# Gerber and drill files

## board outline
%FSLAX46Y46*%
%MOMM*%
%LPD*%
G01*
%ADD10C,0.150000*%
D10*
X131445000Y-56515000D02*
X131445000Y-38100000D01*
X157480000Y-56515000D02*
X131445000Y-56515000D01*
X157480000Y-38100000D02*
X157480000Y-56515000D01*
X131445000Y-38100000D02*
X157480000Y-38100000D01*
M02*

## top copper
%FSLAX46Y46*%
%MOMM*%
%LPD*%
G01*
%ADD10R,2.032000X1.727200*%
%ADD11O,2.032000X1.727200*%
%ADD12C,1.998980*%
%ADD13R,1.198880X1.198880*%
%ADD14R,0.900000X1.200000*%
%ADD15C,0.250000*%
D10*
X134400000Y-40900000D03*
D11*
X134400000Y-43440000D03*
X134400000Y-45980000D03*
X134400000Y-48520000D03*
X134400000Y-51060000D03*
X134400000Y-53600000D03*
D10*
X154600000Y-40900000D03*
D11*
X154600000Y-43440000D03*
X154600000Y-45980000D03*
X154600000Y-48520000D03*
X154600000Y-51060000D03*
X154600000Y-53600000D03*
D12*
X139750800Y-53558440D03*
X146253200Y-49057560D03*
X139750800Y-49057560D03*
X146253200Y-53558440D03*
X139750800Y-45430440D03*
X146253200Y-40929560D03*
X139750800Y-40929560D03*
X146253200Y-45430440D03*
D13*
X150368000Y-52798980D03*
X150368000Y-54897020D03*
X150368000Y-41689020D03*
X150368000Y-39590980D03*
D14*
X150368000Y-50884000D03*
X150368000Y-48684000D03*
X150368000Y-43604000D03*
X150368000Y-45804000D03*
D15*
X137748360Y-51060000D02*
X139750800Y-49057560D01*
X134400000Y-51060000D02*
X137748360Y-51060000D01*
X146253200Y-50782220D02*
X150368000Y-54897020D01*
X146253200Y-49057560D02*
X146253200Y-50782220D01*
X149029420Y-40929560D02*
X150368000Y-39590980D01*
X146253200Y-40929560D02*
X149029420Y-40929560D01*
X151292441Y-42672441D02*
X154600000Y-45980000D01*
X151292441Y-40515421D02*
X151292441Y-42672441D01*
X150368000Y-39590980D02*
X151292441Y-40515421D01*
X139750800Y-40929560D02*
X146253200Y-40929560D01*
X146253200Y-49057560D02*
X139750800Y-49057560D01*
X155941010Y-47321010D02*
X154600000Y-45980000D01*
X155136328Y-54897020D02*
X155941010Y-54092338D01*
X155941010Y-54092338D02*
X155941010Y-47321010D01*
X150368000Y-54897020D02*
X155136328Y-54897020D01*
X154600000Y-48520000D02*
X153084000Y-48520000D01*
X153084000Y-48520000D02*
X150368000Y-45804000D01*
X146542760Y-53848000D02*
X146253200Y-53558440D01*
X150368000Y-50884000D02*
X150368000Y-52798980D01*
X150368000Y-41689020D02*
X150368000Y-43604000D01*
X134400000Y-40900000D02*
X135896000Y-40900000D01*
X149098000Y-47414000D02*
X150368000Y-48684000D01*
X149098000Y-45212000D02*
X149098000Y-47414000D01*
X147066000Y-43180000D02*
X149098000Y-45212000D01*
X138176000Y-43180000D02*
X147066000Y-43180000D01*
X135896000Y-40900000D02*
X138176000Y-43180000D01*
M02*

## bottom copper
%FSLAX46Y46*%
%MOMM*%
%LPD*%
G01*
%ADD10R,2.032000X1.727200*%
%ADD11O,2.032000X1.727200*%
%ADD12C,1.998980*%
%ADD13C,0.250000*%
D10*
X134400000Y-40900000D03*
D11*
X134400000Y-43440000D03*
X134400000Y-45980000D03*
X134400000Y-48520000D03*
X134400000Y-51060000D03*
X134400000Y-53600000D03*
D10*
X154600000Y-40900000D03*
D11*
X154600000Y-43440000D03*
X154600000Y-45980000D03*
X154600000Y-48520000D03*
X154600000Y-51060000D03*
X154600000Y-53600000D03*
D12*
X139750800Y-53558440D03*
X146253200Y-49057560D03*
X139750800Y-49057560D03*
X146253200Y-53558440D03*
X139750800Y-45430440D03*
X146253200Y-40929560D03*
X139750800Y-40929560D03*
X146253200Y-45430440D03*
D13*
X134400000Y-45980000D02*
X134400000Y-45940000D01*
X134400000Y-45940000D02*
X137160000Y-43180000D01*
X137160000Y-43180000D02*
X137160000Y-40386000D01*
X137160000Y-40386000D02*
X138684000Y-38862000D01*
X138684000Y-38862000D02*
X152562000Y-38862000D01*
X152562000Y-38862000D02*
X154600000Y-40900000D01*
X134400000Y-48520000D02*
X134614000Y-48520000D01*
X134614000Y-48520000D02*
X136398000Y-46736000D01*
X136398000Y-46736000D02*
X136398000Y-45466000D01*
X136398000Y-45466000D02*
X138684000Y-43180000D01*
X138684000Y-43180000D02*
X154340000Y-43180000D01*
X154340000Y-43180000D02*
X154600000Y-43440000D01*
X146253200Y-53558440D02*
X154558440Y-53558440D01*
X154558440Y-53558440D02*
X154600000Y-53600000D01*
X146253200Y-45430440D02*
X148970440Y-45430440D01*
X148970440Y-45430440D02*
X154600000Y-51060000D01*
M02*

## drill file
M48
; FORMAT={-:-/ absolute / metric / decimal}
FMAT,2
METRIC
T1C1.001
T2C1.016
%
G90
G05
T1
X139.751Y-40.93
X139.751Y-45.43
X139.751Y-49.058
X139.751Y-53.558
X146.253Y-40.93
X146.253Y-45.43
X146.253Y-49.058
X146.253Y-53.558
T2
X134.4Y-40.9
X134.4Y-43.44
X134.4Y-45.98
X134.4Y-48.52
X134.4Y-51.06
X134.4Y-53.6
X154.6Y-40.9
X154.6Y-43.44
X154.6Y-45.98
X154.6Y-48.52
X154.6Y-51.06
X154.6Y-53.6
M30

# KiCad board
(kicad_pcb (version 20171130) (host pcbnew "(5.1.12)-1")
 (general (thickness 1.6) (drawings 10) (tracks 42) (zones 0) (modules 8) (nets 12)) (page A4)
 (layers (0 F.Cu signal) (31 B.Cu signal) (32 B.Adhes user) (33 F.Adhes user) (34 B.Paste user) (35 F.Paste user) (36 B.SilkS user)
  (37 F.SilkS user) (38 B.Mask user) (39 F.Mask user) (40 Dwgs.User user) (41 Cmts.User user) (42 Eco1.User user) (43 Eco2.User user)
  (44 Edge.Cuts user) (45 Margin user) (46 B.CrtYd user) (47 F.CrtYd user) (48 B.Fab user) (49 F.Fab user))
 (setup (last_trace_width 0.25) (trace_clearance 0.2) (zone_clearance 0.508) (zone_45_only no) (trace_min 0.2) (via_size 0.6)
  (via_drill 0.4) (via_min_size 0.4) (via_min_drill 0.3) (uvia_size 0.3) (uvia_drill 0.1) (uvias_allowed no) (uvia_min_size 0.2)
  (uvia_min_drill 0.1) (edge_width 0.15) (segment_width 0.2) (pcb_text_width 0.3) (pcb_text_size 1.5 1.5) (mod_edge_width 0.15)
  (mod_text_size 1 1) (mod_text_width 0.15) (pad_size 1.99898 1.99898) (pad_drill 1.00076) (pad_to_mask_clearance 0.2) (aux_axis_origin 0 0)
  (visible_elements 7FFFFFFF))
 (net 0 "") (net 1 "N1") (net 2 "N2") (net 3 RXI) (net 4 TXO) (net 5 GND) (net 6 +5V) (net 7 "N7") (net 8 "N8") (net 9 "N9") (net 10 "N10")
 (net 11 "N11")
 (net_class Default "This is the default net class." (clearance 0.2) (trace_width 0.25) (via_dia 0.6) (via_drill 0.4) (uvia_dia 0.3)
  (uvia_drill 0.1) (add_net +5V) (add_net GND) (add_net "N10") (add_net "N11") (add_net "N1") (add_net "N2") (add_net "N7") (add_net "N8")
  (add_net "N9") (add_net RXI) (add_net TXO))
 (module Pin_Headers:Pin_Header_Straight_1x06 (layer F.Cu) (at 134.4 40.9)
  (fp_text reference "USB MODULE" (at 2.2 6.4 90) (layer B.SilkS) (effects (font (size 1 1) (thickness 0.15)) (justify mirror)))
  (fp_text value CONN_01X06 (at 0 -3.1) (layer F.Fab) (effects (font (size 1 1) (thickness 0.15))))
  (pad 1 thru_hole rect (at 0 0) (size 2.032 1.7272) (drill 1.016) (layers *.Cu *.Mask F.SilkS) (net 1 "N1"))
  (pad 2 thru_hole oval (at 0 2.54) (size 2.032 1.7272) (drill 1.016) (layers *.Cu *.Mask F.SilkS) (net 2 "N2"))
  (pad 3 thru_hole oval (at 0 5.08) (size 2.032 1.7272) (drill 1.016) (layers *.Cu *.Mask F.SilkS) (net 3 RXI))
  (pad 4 thru_hole oval (at 0 7.62) (size 2.032 1.7272) (drill 1.016) (layers *.Cu *.Mask F.SilkS) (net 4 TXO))
  (pad 5 thru_hole oval (at 0 10.16) (size 2.032 1.7272) (drill 1.016) (layers *.Cu *.Mask F.SilkS) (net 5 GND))
  (pad 6 thru_hole oval (at 0 12.7) (size 2.032 1.7272) (drill 1.016) (layers *.Cu *.Mask F.SilkS) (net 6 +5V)))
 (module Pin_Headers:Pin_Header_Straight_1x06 (layer F.Cu) (at 154.6 40.9)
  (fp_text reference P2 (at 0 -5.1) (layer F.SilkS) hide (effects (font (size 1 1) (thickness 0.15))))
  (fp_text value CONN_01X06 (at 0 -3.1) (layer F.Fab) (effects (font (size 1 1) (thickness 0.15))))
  (pad 1 thru_hole rect (at 0 0) (size 2.032 1.7272) (drill 1.016) (layers *.Cu *.Mask F.SilkS) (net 3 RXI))
  (pad 2 thru_hole oval (at 0 2.54) (size 2.032 1.7272) (drill 1.016) (layers *.Cu *.Mask F.SilkS) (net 4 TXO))
  (pad 3 thru_hole oval (at 0 5.08) (size 2.032 1.7272) (drill 1.016) (layers *.Cu *.Mask F.SilkS) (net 5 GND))
  (pad 4 thru_hole oval (at 0 7.62) (size 2.032 1.7272) (drill 1.016) (layers *.Cu *.Mask F.SilkS) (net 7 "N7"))
  (pad 5 thru_hole oval (at 0 10.16) (size 2.032 1.7272) (drill 1.016) (layers *.Cu *.Mask F.SilkS) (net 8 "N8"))
  (pad 6 thru_hole oval (at 0 12.7) (size 2.032 1.7272) (drill 1.016) (layers *.Cu *.Mask F.SilkS) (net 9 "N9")))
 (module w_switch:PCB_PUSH (layer F.Cu) (at 143.002 51.308 90)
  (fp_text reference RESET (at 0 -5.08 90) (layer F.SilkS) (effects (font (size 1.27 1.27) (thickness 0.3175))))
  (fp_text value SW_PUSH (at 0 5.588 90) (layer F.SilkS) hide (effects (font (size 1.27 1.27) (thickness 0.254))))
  (pad 1 thru_hole circle (at -2.25044 -3.2512 90) (size 1.99898 1.99898) (drill 1.00076) (layers *.Cu *.Mask F.SilkS))
  (pad 2 thru_hole circle (at 2.25044 3.2512 90) (size 1.99898 1.99898) (drill 1.00076) (layers *.Cu *.Mask F.SilkS) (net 5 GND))
  (pad 4 thru_hole circle (at 2.25044 -3.2512 90) (size 1.99898 1.99898) (drill 1.00076) (layers *.Cu *.Mask F.SilkS) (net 5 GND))
  (pad 3 thru_hole circle (at -2.25044 3.2512 90) (size 1.99898 1.99898) (drill 1.00076) (layers *.Cu *.Mask F.SilkS) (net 9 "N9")))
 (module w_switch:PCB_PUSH (layer F.Cu) (at 143.002 43.18 90)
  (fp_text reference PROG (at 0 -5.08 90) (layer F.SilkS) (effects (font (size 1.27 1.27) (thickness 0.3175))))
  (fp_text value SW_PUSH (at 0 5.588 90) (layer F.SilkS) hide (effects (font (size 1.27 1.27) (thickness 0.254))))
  (pad 1 thru_hole circle (at -2.25044 -3.2512 90) (size 1.99898 1.99898) (drill 1.00076) (layers *.Cu *.Mask F.SilkS))
  (pad 2 thru_hole circle (at 2.25044 3.2512 90) (size 1.99898 1.99898) (drill 1.00076) (layers *.Cu *.Mask F.SilkS) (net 5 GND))
  (pad 4 thru_hole circle (at 2.25044 -3.2512 90) (size 1.99898 1.99898) (drill 1.00076) (layers *.Cu *.Mask F.SilkS) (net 5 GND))
  (pad 3 thru_hole circle (at -2.25044 3.2512 90) (size 1.99898 1.99898) (drill 1.00076) (layers *.Cu *.Mask F.SilkS) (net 8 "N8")))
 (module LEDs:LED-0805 (layer F.Cu) (at 150.368 53.848 90)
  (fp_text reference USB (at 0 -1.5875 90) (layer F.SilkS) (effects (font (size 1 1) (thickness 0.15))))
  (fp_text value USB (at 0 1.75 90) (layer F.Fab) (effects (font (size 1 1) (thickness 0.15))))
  (pad 2 smd rect (at 1.04902 0 270) (size 1.19888 1.19888) (layers F.Cu F.Paste F.Mask) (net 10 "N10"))
  (pad 1 smd rect (at -1.04902 0 270) (size 1.19888 1.19888) (layers F.Cu F.Paste F.Mask) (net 5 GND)))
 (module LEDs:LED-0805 (layer F.Cu) (at 150.368 40.64 270)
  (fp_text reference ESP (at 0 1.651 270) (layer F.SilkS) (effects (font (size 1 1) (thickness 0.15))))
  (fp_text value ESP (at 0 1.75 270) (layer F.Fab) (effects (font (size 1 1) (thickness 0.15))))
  (pad 2 smd rect (at 1.04902 0 90) (size 1.19888 1.19888) (layers F.Cu F.Paste F.Mask) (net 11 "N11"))
  (pad 1 smd rect (at -1.04902 0 90) (size 1.19888 1.19888) (layers F.Cu F.Paste F.Mask) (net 5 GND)))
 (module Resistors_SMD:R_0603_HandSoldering (layer F.Cu) (at 150.368 49.784 90)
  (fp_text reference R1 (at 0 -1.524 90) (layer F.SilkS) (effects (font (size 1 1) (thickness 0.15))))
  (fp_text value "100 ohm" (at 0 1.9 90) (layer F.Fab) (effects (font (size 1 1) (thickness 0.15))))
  (pad 1 smd rect (at -1.1 0 90) (size 1.2 0.9) (layers F.Cu F.Paste F.Mask) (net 10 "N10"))
  (pad 2 smd rect (at 1.1 0 90) (size 1.2 0.9) (layers F.Cu F.Paste F.Mask) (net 1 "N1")))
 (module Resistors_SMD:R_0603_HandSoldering (layer F.Cu) (at 150.368 44.704 270)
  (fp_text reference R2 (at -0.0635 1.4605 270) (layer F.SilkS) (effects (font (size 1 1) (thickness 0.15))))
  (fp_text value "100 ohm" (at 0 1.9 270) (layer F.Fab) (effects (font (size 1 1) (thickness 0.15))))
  (pad 1 smd rect (at -1.1 0 270) (size 1.2 0.9) (layers F.Cu F.Paste F.Mask) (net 11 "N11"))
  (pad 2 smd rect (at 1.1 0 270) (size 1.2 0.9) (layers F.Cu F.Paste F.Mask) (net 7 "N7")))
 (gr_line (start 131.445 56.515) (end 131.445 38.1) (angle 90) (layer Edge.Cuts) (width 0.15))
 (gr_line (start 157.48 56.515) (end 131.445 56.515) (angle 90) (layer Edge.Cuts) (width 0.15))
 (gr_line (start 157.48 38.1) (end 157.48 56.515) (angle 90) (layer Edge.Cuts) (width 0.15))
 (gr_line (start 131.445 38.1) (end 157.48 38.1) (angle 90) (layer Edge.Cuts) (width 0.15))
 (segment (start 134.4 45.98) (end 134.4 45.94) (width 0.25) (layer B.Cu) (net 3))
 (segment (start 134.4 45.94) (end 137.16 43.18) (width 0.25) (layer B.Cu) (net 3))
 (segment (start 137.16 43.18) (end 137.16 40.386) (width 0.25) (layer B.Cu) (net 3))
 (segment (start 137.16 40.386) (end 138.684 38.862) (width 0.25) (layer B.Cu) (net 3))
 (segment (start 138.684 38.862) (end 152.562 38.862) (width 0.25) (layer B.Cu) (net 3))
 (segment (start 152.562 38.862) (end 154.6 40.9) (width 0.25) (layer B.Cu) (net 3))
 (segment (start 134.4 48.52) (end 134.614 48.52) (width 0.25) (layer B.Cu) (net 4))
 (segment (start 134.614 48.52) (end 136.398 46.736) (width 0.25) (layer B.Cu) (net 4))
 (segment (start 136.398 46.736) (end 136.398 45.466) (width 0.25) (layer B.Cu) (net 4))
 (segment (start 136.398 45.466) (end 138.684 43.18) (width 0.25) (layer B.Cu) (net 4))
 (segment (start 138.684 43.18) (end 154.34 43.18) (width 0.25) (layer B.Cu) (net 4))
 (segment (start 154.34 43.18) (end 154.6 43.44) (width 0.25) (layer B.Cu) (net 4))
 (segment (start 137.74836 51.06) (end 139.7508 49.05756) (width 0.25) (layer F.Cu) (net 5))
 (segment (start 134.4 51.06) (end 137.74836 51.06) (width 0.25) (layer F.Cu) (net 5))
 (segment (start 146.2532 50.78222) (end 150.368 54.89702) (width 0.25) (layer F.Cu) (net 5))
 (segment (start 146.2532 49.05756) (end 146.2532 50.78222) (width 0.25) (layer F.Cu) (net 5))
 (segment (start 149.02942 40.92956) (end 150.368 39.59098) (width 0.25) (layer F.Cu) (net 5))
 (segment (start 146.2532 40.92956) (end 149.02942 40.92956) (width 0.25) (layer F.Cu) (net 5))
 (segment (start 151.292441 42.672441) (end 154.6 45.98) (width 0.25) (layer F.Cu) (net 5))
 (segment (start 151.292441 40.515421) (end 151.292441 42.672441) (width 0.25) (layer F.Cu) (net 5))
 (segment (start 150.368 39.59098) (end 151.292441 40.515421) (width 0.25) (layer F.Cu) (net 5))
 (segment (start 139.7508 40.92956) (end 146.2532 40.92956) (width 0.25) (layer F.Cu) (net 5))
 (segment (start 146.2532 49.05756) (end 139.7508 49.05756) (width 0.25) (layer F.Cu) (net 5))
 (segment (start 155.94101 47.32101) (end 154.6 45.98) (width 0.25) (layer F.Cu) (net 5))
 (segment (start 155.136328 54.89702) (end 155.94101 54.092338) (width 0.25) (layer F.Cu) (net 5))
 (segment (start 155.94101 54.092338) (end 155.94101 47.32101) (width 0.25) (layer F.Cu) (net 5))
 (segment (start 150.368 54.89702) (end 155.136328 54.89702) (width 0.25) (layer F.Cu) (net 5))
 (segment (start 154.6 48.52) (end 153.084 48.52) (width 0.25) (layer F.Cu) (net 7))
 (segment (start 153.084 48.52) (end 150.368 45.804) (width 0.25) (layer F.Cu) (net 7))
 (segment (start 146.2532 53.55844) (end 154.55844 53.55844) (width 0.25) (layer B.Cu) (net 9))
 (segment (start 154.55844 53.55844) (end 154.6 53.6) (width 0.25) (layer B.Cu) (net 9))
 (segment (start 146.54276 53.848) (end 146.2532 53.55844) (width 0.25) (layer F.Cu) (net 9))
 (segment (start 146.2532 45.43044) (end 148.97044 45.43044) (width 0.25) (layer B.Cu) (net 8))
 (segment (start 148.97044 45.43044) (end 154.6 51.06) (width 0.25) (layer B.Cu) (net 8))
 (segment (start 150.368 50.884) (end 150.368 52.79898) (width 0.25) (layer F.Cu) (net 10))
 (segment (start 150.368 41.68902) (end 150.368 43.604) (width 0.25) (layer F.Cu) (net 11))
 (segment (start 134.4 40.9) (end 135.896 40.9) (width 0.25) (layer F.Cu) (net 1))
 (segment (start 149.098 47.414) (end 150.368 48.684) (width 0.25) (layer F.Cu) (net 1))
 (segment (start 149.098 45.212) (end 149.098 47.414) (width 0.25) (layer F.Cu) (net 1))
 (segment (start 147.066 43.18) (end 149.098 45.212) (width 0.25) (layer F.Cu) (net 1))
 (segment (start 138.176 43.18) (end 147.066 43.18) (width 0.25) (layer F.Cu) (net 1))
 (segment (start 135.896 40.9) (end 138.176 43.18) (width 0.25) (layer F.Cu) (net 1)))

